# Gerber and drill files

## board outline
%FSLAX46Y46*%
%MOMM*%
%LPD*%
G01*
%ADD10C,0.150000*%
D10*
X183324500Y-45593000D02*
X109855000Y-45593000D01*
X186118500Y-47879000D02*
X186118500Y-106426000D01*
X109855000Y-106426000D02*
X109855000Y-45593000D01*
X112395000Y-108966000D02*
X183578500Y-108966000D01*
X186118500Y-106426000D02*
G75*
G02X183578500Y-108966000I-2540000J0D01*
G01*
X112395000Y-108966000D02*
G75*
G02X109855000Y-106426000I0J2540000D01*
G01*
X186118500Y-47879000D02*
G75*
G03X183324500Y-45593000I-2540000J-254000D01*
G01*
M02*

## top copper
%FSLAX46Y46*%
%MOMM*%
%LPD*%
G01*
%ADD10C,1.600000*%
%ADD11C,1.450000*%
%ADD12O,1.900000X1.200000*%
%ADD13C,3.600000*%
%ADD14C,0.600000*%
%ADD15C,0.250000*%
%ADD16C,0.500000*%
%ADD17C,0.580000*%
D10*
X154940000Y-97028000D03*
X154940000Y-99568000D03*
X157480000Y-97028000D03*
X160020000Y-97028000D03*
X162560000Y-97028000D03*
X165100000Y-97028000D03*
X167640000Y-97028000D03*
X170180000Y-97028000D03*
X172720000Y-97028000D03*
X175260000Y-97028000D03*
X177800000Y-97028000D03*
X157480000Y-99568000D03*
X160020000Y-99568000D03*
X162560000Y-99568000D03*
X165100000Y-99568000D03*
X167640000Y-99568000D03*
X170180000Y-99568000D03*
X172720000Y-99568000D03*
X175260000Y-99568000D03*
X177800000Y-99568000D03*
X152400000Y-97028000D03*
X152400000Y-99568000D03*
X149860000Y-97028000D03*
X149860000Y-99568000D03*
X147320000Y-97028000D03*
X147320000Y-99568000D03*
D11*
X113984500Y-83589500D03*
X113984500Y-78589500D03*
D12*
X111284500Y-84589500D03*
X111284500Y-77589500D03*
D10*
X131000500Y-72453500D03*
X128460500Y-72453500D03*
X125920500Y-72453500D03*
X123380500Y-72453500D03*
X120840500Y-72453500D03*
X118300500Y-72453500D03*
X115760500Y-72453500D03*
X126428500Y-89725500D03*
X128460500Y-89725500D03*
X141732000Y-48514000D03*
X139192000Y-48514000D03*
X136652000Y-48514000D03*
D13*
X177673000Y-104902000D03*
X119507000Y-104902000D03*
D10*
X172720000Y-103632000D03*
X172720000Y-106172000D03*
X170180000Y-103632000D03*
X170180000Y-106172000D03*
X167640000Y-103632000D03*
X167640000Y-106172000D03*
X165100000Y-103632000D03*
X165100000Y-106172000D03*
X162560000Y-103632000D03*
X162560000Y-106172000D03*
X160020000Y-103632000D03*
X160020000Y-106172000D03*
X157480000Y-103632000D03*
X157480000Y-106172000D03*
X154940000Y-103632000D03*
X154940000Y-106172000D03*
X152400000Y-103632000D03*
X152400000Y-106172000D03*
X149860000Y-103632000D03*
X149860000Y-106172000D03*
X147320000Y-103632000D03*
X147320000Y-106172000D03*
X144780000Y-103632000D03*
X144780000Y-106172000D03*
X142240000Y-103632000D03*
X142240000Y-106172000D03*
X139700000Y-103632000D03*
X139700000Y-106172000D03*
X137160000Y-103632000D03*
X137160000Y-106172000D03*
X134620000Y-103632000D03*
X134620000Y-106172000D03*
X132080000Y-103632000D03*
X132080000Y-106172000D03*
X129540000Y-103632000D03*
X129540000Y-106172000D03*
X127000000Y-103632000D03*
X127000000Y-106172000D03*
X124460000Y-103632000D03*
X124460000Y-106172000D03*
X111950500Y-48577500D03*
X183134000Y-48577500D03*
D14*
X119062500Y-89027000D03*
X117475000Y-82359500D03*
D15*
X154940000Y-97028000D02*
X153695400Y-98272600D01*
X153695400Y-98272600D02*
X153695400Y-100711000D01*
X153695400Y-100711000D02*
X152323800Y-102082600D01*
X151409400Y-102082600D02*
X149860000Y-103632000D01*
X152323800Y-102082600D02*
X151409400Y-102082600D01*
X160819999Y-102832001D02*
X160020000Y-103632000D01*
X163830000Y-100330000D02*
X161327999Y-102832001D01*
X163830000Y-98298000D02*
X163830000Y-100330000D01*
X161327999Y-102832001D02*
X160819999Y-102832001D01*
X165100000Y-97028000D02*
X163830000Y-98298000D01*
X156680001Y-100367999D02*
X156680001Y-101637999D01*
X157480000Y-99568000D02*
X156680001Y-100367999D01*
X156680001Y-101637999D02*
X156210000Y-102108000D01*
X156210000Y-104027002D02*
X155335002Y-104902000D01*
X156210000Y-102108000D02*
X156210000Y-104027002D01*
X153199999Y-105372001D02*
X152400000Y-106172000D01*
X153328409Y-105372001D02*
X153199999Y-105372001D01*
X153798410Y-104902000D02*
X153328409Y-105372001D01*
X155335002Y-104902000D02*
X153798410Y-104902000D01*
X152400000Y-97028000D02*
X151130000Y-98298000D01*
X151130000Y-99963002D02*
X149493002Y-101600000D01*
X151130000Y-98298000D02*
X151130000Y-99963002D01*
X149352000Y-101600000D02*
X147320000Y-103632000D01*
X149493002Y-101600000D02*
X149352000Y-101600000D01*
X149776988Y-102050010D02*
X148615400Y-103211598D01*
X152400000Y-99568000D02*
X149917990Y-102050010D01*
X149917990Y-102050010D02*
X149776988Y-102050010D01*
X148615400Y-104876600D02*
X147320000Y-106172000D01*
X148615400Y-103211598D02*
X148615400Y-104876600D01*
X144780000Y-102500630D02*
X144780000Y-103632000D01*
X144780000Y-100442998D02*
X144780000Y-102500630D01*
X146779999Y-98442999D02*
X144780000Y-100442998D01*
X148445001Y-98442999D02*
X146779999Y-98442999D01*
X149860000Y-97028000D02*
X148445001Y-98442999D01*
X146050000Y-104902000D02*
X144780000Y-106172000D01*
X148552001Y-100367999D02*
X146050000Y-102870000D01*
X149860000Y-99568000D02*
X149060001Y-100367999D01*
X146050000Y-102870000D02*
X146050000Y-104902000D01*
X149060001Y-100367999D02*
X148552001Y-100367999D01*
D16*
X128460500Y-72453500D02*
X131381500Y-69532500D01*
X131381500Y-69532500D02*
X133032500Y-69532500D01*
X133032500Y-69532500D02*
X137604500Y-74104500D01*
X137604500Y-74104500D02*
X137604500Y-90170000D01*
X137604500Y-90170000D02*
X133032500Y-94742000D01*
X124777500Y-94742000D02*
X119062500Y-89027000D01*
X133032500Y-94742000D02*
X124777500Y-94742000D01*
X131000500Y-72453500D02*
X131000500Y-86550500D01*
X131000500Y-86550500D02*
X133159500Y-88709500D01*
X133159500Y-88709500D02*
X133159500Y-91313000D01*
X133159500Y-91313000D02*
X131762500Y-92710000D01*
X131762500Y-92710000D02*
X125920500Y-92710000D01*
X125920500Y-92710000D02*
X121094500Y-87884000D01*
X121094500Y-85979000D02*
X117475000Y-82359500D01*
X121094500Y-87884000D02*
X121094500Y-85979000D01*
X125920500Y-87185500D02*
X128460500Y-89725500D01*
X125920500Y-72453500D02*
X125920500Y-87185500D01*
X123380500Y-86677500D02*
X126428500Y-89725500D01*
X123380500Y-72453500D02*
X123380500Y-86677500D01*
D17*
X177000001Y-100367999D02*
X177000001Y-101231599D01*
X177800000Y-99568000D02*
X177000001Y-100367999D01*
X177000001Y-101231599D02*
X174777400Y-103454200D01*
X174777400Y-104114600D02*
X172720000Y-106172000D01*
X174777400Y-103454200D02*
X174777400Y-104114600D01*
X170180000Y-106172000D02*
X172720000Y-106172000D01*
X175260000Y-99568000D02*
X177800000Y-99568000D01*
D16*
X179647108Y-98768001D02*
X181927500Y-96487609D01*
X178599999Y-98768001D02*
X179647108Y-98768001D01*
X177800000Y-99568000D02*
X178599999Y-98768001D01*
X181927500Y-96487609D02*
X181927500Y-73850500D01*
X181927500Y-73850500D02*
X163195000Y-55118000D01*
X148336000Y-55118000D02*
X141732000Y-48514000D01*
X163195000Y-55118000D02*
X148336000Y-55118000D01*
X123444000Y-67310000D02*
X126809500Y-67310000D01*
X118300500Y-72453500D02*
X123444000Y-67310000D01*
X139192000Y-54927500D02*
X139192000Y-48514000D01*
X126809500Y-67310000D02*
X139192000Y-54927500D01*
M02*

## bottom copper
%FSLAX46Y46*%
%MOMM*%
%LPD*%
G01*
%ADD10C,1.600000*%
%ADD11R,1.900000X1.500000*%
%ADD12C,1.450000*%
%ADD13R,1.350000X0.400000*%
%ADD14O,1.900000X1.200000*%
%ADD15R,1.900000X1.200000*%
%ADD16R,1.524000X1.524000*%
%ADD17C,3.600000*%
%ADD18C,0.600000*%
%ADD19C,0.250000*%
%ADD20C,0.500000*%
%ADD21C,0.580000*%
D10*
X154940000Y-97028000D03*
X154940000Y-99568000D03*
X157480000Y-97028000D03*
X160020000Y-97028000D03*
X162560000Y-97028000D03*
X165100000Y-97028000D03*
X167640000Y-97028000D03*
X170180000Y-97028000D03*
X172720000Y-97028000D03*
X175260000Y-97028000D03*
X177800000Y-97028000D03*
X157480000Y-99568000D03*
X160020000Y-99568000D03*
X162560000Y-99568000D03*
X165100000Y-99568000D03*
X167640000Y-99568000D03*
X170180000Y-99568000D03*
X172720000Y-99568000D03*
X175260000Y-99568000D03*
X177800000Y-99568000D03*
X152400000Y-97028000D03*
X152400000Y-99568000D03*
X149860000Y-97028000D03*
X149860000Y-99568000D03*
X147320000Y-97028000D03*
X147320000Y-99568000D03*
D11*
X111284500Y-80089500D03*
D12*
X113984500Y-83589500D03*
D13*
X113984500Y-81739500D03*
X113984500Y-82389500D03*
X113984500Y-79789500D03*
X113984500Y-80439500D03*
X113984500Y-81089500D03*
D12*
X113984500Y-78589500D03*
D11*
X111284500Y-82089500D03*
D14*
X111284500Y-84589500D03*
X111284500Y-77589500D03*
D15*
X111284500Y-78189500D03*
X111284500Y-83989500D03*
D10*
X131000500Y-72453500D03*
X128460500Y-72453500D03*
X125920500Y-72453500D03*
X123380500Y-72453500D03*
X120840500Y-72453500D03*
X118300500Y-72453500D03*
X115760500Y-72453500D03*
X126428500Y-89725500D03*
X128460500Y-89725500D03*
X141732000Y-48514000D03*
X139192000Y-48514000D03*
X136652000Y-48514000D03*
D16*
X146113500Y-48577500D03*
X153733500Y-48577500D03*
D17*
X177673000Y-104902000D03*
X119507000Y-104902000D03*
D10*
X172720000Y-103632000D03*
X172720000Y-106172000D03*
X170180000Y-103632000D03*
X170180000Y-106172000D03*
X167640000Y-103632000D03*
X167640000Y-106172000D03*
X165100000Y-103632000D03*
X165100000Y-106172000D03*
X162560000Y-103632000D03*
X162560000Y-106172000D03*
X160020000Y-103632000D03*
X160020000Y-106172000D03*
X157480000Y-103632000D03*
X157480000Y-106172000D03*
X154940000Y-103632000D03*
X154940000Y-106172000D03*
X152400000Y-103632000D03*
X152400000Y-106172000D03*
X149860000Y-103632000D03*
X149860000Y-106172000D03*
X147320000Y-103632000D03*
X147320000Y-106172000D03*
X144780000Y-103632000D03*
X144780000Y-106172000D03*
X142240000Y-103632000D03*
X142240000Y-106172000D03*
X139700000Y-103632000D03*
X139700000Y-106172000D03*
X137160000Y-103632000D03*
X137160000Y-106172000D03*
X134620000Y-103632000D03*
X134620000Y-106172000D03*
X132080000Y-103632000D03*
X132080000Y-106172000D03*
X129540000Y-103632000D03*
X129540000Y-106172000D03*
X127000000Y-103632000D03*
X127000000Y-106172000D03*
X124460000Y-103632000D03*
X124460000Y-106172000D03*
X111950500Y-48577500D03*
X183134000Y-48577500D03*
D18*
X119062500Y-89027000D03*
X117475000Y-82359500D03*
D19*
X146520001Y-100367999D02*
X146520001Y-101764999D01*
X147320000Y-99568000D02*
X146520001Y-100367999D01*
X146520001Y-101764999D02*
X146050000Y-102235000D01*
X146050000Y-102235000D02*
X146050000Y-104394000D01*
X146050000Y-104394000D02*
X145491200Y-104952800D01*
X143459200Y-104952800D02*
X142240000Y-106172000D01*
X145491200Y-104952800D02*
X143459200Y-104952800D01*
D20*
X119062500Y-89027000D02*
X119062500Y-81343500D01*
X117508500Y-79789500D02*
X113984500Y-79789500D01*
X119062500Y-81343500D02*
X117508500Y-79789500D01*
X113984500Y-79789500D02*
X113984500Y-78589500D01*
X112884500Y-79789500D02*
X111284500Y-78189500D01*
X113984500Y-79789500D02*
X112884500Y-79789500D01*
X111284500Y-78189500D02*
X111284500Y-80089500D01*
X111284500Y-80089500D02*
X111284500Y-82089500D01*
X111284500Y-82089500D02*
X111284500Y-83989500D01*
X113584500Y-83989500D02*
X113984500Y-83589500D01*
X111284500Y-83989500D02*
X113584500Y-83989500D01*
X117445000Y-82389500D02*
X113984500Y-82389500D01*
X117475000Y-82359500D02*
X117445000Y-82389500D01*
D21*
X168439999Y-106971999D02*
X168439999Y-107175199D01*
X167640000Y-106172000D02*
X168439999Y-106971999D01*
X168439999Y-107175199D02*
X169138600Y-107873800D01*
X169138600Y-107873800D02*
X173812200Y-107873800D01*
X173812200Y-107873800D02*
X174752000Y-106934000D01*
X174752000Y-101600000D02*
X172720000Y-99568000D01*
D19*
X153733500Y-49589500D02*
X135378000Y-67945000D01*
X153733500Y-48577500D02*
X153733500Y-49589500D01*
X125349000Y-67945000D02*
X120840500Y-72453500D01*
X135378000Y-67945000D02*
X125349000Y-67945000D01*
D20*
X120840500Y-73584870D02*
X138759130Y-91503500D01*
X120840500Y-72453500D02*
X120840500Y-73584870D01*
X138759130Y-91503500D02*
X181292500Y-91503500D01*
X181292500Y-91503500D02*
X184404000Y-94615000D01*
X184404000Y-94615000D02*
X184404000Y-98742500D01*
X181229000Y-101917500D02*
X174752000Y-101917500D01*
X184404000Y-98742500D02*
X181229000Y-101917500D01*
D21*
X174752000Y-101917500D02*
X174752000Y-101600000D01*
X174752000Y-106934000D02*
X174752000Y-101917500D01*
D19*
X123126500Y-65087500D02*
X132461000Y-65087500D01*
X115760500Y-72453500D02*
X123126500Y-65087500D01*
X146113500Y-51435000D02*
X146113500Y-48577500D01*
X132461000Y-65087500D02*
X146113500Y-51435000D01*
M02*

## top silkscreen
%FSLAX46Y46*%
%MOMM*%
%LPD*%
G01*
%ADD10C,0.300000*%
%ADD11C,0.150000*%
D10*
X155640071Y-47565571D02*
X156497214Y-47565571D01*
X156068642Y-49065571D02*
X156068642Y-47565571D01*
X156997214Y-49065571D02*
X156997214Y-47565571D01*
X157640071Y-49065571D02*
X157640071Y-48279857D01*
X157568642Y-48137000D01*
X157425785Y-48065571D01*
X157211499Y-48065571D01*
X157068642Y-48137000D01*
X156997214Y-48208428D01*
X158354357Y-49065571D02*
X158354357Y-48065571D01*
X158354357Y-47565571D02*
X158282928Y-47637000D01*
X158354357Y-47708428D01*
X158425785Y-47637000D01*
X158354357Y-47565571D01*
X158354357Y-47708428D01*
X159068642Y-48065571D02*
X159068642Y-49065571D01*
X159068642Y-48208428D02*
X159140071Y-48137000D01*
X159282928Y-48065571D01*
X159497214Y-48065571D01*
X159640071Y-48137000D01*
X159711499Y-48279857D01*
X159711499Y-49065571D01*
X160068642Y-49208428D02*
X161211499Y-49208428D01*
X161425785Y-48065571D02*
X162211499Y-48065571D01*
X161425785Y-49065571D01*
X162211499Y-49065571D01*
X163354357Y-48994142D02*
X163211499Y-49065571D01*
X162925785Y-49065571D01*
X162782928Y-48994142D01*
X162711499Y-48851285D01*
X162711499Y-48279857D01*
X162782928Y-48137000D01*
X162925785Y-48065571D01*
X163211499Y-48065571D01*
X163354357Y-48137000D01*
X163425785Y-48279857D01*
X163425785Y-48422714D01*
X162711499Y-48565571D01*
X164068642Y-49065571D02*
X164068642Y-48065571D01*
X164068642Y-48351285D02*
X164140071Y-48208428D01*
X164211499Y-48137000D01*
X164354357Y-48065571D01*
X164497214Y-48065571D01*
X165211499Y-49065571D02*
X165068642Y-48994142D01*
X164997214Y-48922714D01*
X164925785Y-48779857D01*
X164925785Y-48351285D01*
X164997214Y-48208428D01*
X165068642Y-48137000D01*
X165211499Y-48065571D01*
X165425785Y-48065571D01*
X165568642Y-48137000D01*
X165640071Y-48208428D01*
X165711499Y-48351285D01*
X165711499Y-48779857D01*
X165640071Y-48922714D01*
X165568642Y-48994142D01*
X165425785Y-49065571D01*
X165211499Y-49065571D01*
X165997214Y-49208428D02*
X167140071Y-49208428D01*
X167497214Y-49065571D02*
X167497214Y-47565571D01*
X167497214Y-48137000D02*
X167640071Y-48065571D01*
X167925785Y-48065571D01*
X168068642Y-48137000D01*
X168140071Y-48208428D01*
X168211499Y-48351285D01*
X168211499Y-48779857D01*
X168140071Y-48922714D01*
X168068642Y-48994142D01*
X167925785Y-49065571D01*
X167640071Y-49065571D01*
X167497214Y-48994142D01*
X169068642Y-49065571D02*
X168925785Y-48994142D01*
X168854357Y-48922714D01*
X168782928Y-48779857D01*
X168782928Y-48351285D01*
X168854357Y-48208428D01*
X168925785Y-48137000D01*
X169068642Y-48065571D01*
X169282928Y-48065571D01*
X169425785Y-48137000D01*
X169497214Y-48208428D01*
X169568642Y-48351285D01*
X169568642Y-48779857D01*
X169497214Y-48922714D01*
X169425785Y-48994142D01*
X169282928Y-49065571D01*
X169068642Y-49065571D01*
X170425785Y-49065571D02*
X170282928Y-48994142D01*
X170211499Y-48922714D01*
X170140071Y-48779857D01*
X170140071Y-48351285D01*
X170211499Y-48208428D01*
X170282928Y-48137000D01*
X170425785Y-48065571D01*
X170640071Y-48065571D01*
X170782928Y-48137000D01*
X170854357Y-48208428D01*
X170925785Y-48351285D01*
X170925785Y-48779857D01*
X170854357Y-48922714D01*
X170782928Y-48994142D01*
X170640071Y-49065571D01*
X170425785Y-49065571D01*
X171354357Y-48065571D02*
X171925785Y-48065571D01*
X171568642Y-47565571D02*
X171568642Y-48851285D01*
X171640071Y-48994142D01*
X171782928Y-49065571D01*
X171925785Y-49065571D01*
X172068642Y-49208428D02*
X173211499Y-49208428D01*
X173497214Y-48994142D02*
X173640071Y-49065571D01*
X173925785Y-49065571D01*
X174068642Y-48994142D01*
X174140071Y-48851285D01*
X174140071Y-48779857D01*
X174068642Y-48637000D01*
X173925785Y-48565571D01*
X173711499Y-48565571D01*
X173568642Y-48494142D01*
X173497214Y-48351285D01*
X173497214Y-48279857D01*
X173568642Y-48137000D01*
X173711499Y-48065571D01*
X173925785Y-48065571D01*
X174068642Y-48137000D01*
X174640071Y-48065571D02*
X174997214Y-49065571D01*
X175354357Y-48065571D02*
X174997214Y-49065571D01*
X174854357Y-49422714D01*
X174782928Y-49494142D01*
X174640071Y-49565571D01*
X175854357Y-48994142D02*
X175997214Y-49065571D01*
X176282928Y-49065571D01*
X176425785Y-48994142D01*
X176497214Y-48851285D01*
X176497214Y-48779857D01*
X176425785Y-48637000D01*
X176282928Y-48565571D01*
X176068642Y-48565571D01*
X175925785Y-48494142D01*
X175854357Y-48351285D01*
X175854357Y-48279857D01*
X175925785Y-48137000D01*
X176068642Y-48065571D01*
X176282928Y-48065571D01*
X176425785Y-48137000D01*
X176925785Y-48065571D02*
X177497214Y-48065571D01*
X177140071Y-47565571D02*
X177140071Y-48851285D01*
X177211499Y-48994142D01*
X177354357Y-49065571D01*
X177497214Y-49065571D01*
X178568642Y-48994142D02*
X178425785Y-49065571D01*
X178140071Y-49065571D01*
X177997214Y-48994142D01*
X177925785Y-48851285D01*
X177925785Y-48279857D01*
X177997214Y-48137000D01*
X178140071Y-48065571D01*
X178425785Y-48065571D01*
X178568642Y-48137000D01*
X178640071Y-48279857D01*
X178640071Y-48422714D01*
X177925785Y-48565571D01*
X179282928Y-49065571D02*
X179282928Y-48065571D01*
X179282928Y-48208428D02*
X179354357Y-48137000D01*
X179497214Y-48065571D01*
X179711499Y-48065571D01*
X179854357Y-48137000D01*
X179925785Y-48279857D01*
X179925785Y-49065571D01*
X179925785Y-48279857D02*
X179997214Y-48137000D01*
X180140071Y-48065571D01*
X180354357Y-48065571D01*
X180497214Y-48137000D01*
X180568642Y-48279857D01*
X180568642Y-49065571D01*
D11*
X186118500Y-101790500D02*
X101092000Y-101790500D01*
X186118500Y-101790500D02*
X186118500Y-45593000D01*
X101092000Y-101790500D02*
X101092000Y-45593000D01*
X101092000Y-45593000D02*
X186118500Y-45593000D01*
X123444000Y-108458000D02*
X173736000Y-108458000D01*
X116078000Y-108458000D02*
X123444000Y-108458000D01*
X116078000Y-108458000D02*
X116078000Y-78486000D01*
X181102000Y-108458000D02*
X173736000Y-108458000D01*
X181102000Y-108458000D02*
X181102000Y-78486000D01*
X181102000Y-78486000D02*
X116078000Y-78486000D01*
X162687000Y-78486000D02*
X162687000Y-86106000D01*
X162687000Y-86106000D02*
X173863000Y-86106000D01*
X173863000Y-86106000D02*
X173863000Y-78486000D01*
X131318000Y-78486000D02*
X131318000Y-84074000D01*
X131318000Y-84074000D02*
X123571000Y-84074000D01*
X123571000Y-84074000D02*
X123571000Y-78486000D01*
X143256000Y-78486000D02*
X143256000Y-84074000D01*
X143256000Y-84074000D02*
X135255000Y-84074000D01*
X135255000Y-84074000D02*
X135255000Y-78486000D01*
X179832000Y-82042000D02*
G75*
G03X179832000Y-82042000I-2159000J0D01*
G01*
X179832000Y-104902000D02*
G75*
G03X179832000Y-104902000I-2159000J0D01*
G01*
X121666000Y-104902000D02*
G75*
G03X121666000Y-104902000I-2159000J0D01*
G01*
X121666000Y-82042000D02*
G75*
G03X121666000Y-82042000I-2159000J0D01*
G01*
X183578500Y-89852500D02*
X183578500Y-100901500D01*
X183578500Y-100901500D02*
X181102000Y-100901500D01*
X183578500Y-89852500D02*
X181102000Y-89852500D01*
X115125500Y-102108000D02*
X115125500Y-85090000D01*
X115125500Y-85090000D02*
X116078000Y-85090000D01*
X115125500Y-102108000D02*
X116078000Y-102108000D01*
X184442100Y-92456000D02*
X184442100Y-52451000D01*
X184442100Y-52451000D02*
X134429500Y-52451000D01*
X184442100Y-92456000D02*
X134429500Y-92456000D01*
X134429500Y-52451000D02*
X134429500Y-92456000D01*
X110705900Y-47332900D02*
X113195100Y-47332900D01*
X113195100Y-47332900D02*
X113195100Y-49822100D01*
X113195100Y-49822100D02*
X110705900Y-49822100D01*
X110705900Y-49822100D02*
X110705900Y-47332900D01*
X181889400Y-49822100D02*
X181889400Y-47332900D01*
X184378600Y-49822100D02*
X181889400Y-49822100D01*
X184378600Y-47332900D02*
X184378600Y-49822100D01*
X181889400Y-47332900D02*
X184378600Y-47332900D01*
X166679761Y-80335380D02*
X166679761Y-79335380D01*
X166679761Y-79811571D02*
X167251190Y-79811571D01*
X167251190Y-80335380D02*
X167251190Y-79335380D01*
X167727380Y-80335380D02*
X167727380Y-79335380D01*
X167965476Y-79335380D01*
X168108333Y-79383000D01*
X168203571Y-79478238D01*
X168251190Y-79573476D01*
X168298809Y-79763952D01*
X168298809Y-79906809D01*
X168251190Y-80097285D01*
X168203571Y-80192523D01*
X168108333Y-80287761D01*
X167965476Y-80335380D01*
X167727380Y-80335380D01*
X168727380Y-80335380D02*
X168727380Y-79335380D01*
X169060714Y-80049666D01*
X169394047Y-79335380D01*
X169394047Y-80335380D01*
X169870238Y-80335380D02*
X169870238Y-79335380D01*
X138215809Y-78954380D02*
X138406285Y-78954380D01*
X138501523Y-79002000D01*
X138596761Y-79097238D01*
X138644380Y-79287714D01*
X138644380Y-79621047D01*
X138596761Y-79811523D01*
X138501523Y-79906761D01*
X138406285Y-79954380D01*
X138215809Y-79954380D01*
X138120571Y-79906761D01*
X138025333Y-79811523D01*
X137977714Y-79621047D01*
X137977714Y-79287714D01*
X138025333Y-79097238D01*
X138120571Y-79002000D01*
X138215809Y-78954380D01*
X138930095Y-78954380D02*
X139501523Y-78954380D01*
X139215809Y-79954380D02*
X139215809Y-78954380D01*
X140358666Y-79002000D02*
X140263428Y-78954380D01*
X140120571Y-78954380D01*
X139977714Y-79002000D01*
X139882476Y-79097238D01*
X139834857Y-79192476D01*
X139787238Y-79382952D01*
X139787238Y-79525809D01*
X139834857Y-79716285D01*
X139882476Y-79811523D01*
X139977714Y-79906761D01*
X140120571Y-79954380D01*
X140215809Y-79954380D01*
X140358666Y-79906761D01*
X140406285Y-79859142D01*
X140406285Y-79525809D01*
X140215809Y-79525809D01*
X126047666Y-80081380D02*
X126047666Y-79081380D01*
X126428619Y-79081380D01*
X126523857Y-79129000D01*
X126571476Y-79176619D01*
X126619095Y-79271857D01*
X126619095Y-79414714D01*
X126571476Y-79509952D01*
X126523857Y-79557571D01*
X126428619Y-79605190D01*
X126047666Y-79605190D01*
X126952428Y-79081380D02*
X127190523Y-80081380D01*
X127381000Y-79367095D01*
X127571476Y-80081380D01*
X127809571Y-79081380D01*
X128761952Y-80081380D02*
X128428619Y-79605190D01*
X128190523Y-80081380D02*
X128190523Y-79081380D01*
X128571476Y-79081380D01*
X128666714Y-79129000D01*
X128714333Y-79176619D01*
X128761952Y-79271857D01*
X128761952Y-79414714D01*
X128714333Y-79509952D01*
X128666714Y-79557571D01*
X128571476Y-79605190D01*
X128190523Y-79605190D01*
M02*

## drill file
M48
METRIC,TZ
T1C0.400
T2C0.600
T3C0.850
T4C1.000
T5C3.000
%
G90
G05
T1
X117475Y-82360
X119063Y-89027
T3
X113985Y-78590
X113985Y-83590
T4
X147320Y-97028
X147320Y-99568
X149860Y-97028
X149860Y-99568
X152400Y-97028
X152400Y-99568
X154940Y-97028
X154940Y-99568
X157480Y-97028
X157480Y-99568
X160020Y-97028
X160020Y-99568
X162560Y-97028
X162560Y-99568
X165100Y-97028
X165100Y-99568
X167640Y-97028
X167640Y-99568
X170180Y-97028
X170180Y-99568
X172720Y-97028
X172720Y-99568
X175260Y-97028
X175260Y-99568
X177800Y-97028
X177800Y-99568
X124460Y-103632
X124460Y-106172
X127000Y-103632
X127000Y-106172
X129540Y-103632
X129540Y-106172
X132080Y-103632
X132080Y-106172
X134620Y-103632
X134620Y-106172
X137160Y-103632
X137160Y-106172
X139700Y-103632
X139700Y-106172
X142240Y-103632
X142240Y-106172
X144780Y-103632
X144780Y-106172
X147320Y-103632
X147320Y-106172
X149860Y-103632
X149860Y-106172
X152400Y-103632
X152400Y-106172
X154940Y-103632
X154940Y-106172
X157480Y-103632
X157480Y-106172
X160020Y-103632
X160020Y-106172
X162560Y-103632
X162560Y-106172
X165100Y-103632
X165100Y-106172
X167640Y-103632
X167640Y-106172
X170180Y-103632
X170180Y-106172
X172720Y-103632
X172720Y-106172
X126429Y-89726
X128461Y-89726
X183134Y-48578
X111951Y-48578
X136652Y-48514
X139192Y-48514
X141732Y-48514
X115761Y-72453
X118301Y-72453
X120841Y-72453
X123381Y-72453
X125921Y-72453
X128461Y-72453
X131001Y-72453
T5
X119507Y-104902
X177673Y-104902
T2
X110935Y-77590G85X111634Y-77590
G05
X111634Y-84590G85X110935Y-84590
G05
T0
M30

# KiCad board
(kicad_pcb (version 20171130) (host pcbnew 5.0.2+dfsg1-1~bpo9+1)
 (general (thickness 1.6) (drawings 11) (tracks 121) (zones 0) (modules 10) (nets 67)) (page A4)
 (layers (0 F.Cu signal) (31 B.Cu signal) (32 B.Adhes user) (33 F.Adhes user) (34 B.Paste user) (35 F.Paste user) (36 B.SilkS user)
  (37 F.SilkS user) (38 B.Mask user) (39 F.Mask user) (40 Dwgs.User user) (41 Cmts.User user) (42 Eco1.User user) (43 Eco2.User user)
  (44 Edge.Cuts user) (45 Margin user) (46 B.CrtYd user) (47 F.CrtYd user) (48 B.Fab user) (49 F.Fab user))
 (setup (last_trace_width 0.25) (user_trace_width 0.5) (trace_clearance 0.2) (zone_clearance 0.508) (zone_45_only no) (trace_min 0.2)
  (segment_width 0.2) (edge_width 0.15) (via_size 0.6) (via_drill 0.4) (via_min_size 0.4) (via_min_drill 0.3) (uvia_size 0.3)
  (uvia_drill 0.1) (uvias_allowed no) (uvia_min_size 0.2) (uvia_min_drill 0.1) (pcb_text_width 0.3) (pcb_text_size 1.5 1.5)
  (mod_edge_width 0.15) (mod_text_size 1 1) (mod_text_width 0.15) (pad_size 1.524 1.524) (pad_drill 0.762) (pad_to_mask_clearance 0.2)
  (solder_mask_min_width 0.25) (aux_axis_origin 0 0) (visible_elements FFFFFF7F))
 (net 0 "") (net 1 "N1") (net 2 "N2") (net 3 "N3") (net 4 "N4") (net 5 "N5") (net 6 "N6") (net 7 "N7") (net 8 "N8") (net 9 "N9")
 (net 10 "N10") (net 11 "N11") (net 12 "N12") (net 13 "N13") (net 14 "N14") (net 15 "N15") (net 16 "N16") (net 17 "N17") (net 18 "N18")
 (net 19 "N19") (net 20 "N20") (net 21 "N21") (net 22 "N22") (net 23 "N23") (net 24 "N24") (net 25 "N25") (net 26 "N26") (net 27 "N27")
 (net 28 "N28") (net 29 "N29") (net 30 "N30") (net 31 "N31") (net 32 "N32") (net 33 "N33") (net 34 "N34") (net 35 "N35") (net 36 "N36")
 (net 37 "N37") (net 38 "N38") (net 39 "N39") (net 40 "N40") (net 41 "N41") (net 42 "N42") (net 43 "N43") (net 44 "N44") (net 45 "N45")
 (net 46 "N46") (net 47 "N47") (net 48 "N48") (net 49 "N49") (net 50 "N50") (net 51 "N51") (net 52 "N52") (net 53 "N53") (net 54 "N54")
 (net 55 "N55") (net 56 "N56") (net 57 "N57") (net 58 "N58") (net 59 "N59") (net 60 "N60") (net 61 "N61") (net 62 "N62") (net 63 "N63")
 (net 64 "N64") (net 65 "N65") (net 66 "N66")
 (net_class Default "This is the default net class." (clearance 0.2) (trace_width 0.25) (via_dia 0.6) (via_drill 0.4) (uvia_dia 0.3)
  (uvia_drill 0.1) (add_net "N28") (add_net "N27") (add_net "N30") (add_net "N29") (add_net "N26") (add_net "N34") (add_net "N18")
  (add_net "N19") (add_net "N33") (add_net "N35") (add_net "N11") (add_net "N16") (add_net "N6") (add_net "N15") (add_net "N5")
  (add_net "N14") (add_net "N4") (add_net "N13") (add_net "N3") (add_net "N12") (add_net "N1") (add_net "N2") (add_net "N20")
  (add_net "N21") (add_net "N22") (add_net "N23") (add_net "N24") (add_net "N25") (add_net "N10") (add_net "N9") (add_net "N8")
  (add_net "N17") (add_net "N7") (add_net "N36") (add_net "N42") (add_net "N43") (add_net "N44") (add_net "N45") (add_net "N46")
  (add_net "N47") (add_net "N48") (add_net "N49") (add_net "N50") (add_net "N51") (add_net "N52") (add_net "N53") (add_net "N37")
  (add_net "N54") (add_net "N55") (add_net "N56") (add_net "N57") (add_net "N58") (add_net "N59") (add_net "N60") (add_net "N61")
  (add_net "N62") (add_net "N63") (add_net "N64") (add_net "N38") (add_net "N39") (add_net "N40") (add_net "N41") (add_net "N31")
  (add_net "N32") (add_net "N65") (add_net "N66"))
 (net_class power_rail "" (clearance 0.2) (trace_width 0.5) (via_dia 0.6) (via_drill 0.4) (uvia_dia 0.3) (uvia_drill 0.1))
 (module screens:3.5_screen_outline (layer F.Cu) (at 162.56 98.298)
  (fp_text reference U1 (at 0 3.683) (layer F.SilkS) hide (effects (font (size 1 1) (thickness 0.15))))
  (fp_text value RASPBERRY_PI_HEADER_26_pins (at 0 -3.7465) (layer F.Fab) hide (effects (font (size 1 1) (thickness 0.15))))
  (fp_line (start 23.5585 3.4925) (end -61.468 3.4925) (layer F.SilkS) (width 0.15))
  (fp_line (start 23.5585 3.4925) (end 23.5585 -52.705) (layer F.SilkS) (width 0.15))
  (fp_line (start -61.468 3.4925) (end -61.468 -52.705) (layer F.SilkS) (width 0.15))
  (fp_line (start -61.468 -52.705) (end 23.5585 -52.705) (layer F.SilkS) (width 0.15))
  (pad 19 thru_hole circle (at -7.62 -1.27) (size 1.6 1.6) (drill 1) (layers *.Cu *.Mask) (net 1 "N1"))
  (pad 20 thru_hole circle (at -7.62 1.27) (size 1.6 1.6) (drill 1) (layers *.Cu *.Mask) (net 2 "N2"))
  (pad 17 thru_hole circle (at -5.08 -1.27) (size 1.6 1.6) (drill 1) (layers *.Cu *.Mask) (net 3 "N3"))
  (pad 15 thru_hole circle (at -2.54 -1.27) (size 1.6 1.6) (drill 1) (layers *.Cu *.Mask) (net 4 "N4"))
  (pad 13 thru_hole circle (at 0 -1.27) (size 1.6 1.6) (drill 1) (layers *.Cu *.Mask) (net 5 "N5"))
  (pad 11 thru_hole circle (at 2.54 -1.27) (size 1.6 1.6) (drill 1) (layers *.Cu *.Mask) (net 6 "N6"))
  (pad 9 thru_hole circle (at 5.08 -1.27) (size 1.6 1.6) (drill 1) (layers *.Cu *.Mask) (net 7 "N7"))
  (pad 7 thru_hole circle (at 7.62 -1.27) (size 1.6 1.6) (drill 1) (layers *.Cu *.Mask) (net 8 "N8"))
  (pad 5 thru_hole circle (at 10.16 -1.27) (size 1.6 1.6) (drill 1) (layers *.Cu *.Mask) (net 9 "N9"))
  (pad 3 thru_hole circle (at 12.7 -1.27) (size 1.6 1.6) (drill 1) (layers *.Cu *.Mask) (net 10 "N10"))
  (pad 1 thru_hole circle (at 15.24 -1.27) (size 1.6 1.6) (drill 1) (layers *.Cu *.Mask) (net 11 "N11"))
  (pad 18 thru_hole circle (at -5.08 1.27) (size 1.6 1.6) (drill 1) (layers *.Cu *.Mask) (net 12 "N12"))
  (pad 16 thru_hole circle (at -2.54 1.27) (size 1.6 1.6) (drill 1) (layers *.Cu *.Mask) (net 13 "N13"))
  (pad 14 thru_hole circle (at 0 1.27) (size 1.6 1.6) (drill 1) (layers *.Cu *.Mask) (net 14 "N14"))
  (pad 12 thru_hole circle (at 2.54 1.27) (size 1.6 1.6) (drill 1) (layers *.Cu *.Mask) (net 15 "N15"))
  (pad 10 thru_hole circle (at 5.08 1.27) (size 1.6 1.6) (drill 1) (layers *.Cu *.Mask) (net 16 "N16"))
  (pad 8 thru_hole circle (at 7.62 1.27) (size 1.6 1.6) (drill 1) (layers *.Cu *.Mask) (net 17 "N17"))
  (pad 6 thru_hole circle (at 10.16 1.27) (size 1.6 1.6) (drill 1) (layers *.Cu *.Mask) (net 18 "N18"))
  (pad 4 thru_hole circle (at 12.7 1.27) (size 1.6 1.6) (drill 1) (layers *.Cu *.Mask) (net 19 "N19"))
  (pad 2 thru_hole circle (at 15.24 1.27) (size 1.6 1.6) (drill 1) (layers *.Cu *.Mask) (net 19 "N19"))
  (pad 21 thru_hole circle (at -10.16 -1.27) (size 1.6 1.6) (drill 1) (layers *.Cu *.Mask) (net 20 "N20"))
  (pad 22 thru_hole circle (at -10.16 1.27) (size 1.6 1.6) (drill 1) (layers *.Cu *.Mask) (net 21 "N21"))
  (pad 23 thru_hole circle (at -12.7 -1.27) (size 1.6 1.6) (drill 1) (layers *.Cu *.Mask) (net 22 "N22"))
  (pad 24 thru_hole circle (at -12.7 1.27) (size 1.6 1.6) (drill 1) (layers *.Cu *.Mask) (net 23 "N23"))
  (pad 25 thru_hole circle (at -15.24 -1.27) (size 1.6 1.6) (drill 1) (layers *.Cu *.Mask) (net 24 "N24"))
  (pad 26 thru_hole circle (at -15.24 1.27) (size 1.6 1.6) (drill 1) (layers *.Cu *.Mask) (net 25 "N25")))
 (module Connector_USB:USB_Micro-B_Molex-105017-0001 (layer B.Cu) (at 112.522 81.0895 90)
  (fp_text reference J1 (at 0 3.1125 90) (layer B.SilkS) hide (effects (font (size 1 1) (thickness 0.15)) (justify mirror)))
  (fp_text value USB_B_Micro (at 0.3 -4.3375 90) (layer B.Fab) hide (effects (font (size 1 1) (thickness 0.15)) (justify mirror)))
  (pad 6 smd rect (at 1 -1.2375 90) (size 1.5 1.9) (layers B.Cu B.Paste B.Mask) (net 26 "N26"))
  (pad 6 thru_hole circle (at -2.5 1.4625 90) (size 1.45 1.45) (drill 0.85) (layers *.Cu *.Mask) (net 26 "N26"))
  (pad 2 smd rect (at -0.65 1.4625 90) (size 0.4 1.35) (layers B.Cu B.Paste B.Mask) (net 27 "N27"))
  (pad 1 smd rect (at -1.3 1.4625 90) (size 0.4 1.35) (layers B.Cu B.Paste B.Mask) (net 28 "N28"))
  (pad 5 smd rect (at 1.3 1.4625 90) (size 0.4 1.35) (layers B.Cu B.Paste B.Mask) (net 26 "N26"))
  (pad 4 smd rect (at 0.65 1.4625 90) (size 0.4 1.35) (layers B.Cu B.Paste B.Mask) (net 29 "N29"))
  (pad 3 smd rect (at 0 1.4625 90) (size 0.4 1.35) (layers B.Cu B.Paste B.Mask) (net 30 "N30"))
  (pad 6 thru_hole circle (at 2.5 1.4625 90) (size 1.45 1.45) (drill 0.85) (layers *.Cu *.Mask) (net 26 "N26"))
  (pad 6 smd rect (at -1 -1.2375 90) (size 1.5 1.9) (layers B.Cu B.Paste B.Mask) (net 26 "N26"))
  (pad 6 thru_hole oval (at -3.5 -1.2375 270) (size 1.2 1.9) (drill oval 0.6 1.3) (layers *.Cu *.Mask) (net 26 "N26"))
  (pad 6 thru_hole oval (at 3.5 -1.2375 90) (size 1.2 1.9) (drill oval 0.6 1.3) (layers *.Cu *.Mask) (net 26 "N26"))
  (pad 6 smd rect (at 2.9 -1.2375 90) (size 1.2 1.9) (layers B.Cu B.Mask) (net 26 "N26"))
  (pad 6 smd rect (at -2.9 -1.2375 90) (size 1.2 1.9) (layers B.Cu B.Mask) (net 26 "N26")))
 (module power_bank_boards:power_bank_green (layer B.Cu) (at 123.3805 72.4535 180)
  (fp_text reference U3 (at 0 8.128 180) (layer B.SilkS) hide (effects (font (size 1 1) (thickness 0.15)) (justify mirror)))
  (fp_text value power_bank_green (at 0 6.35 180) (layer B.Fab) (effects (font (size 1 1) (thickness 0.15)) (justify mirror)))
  (pad 1 thru_hole circle (at -7.62 0 180) (size 1.6 1.6) (drill 1) (layers *.Cu *.Mask) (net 28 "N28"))
  (pad 2 thru_hole circle (at -5.08 0 180) (size 1.6 1.6) (drill 1) (layers *.Cu *.Mask) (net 26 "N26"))
  (pad 3 thru_hole circle (at -2.54 0 180) (size 1.6 1.6) (drill 1) (layers *.Cu *.Mask) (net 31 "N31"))
  (pad 4 thru_hole circle (at 0 0 180) (size 1.6 1.6) (drill 1) (layers *.Cu *.Mask) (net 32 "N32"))
  (pad 5 thru_hole circle (at 2.54 0 180) (size 1.6 1.6) (drill 1) (layers *.Cu *.Mask) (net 18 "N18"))
  (pad 6 thru_hole circle (at 5.08 0 180) (size 1.6 1.6) (drill 1) (layers *.Cu *.Mask) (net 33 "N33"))
  (pad 7 thru_hole circle (at 7.62 0 180) (size 1.6 1.6) (drill 1) (layers *.Cu *.Mask) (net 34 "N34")))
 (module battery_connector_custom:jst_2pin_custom (layer B.Cu) (at 127.4445 89.7255)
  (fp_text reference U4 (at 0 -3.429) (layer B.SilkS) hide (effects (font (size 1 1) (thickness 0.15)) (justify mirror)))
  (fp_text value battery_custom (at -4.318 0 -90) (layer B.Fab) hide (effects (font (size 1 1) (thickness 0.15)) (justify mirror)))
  (pad 1 thru_hole circle (at -1.016 0) (size 1.6 1.6) (drill 1) (layers *.Cu *.Mask) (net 32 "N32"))
  (pad 2 thru_hole circle (at 1.016 0) (size 1.6 1.6) (drill 1) (layers *.Cu *.Mask) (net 31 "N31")))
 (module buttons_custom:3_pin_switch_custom (layer B.Cu) (at 139.192 48.514 180)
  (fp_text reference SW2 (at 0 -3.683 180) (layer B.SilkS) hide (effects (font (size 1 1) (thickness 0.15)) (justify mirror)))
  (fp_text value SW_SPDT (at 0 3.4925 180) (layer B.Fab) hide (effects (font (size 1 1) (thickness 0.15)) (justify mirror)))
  (pad 1 thru_hole circle (at -2.54 0 180) (size 1.6 1.6) (drill 1) (layers *.Cu *.Mask) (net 19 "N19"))
  (pad 2 thru_hole circle (at 0 0 180) (size 1.6 1.6) (drill 1) (layers *.Cu *.Mask) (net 33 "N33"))
  (pad 3 thru_hole circle (at 2.54 0 180) (size 1.6 1.6) (drill 1) (layers *.Cu *.Mask) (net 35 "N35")))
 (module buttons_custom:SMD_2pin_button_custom (layer B.Cu) (at 149.9235 48.5775 180)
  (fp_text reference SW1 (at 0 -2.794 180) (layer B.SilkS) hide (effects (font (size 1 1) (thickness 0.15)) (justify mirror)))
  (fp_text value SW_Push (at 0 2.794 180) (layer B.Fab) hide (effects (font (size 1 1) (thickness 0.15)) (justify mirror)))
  (pad 1 smd rect (at 3.81 0 180) (size 1.524 1.524) (layers B.Cu B.Paste B.Mask) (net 34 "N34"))
  (pad 2 smd rect (at -3.81 0 180) (size 1.524 1.524) (layers B.Cu B.Paste B.Mask) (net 18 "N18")))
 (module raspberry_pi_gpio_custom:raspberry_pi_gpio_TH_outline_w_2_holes (layer F.Cu) (at 148.59 104.902)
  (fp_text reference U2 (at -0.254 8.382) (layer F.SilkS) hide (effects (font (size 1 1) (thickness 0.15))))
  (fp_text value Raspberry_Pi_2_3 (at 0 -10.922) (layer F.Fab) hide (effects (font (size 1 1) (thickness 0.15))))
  (fp_line (start -25.146 3.556) (end 25.146 3.556) (layer F.SilkS) (width 0.15))
  (fp_line (start -32.512 3.556) (end -25.146 3.556) (layer F.SilkS) (width 0.15))
  (fp_line (start -32.512 3.556) (end -32.512 -26.416) (layer F.SilkS) (width 0.15))
  (fp_line (start 32.512 3.556) (end 25.146 3.556) (layer F.SilkS) (width 0.15))
  (fp_line (start 32.512 3.556) (end 32.512 -26.416) (layer F.SilkS) (width 0.15))
  (fp_line (start 32.512 -26.416) (end -32.512 -26.416) (layer F.SilkS) (width 0.15))
  (fp_line (start 14.097 -26.416) (end 14.097 -18.796) (layer F.SilkS) (width 0.15))
  (fp_line (start 14.097 -18.796) (end 25.273 -18.796) (layer F.SilkS) (width 0.15))
  (fp_line (start 25.273 -18.796) (end 25.273 -26.416) (layer F.SilkS) (width 0.15))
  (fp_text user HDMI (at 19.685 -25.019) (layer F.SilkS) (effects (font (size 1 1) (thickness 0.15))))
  (fp_line (start -17.272 -26.416) (end -17.272 -20.828) (layer F.SilkS) (width 0.15))
  (fp_line (start -17.272 -20.828) (end -25.019 -20.828) (layer F.SilkS) (width 0.15))
  (fp_line (start -25.019 -20.828) (end -25.019 -26.416) (layer F.SilkS) (width 0.15))
  (fp_line (start -5.334 -26.416) (end -5.334 -20.828) (layer F.SilkS) (width 0.15))
  (fp_line (start -5.334 -20.828) (end -13.335 -20.828) (layer F.SilkS) (width 0.15))
  (fp_line (start -13.335 -20.828) (end -13.335 -26.416) (layer F.SilkS) (width 0.15))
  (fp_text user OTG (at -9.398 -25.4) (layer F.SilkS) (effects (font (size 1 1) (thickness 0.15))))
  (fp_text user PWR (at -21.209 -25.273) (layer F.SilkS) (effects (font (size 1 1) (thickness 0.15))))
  (fp_circle (center 29.083 -22.86) (end 31.242 -22.86) (layer F.SilkS) (width 0.15))
  (fp_circle (center 29.083 0) (end 31.242 0) (layer F.SilkS) (width 0.15))
  (fp_circle (center -29.083 0) (end -26.924 0) (layer F.SilkS) (width 0.15))
  (fp_circle (center -29.083 -22.86) (end -26.924 -22.86) (layer F.SilkS) (width 0.15))
  (fp_line (start 34.9885 -15.0495) (end 34.9885 -4.0005) (layer F.SilkS) (width 0.15))
  (fp_line (start 34.9885 -4.0005) (end 32.512 -4.0005) (layer F.SilkS) (width 0.15))
  (fp_line (start 34.9885 -15.0495) (end 32.512 -15.0495) (layer F.SilkS) (width 0.15))
  (fp_line (start -33.4645 -2.794) (end -33.4645 -19.812) (layer F.SilkS) (width 0.15))
  (fp_line (start -33.4645 -19.812) (end -32.512 -19.812) (layer F.SilkS) (width 0.15))
  (fp_line (start -33.4645 -2.794) (end -32.512 -2.794) (layer F.SilkS) (width 0.15))
  (pad 0 thru_hole circle (at 29.083 0) (size 3.6 3.6) (drill 3) (layers *.Cu *.Mask))
  (pad 0 thru_hole circle (at -29.083 0) (size 3.6 3.6) (drill 3) (layers *.Cu *.Mask))
  (pad 1 thru_hole circle (at 24.13 -1.27 180) (size 1.6 1.6) (drill 1) (layers *.Cu *.Mask) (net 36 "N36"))
  (pad 2 thru_hole circle (at 24.13 1.27 180) (size 1.6 1.6) (drill 1) (layers *.Cu *.Mask) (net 19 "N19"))
  (pad 3 thru_hole circle (at 21.59 -1.27 180) (size 1.6 1.6) (drill 1) (layers *.Cu *.Mask) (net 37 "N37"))
  (pad 4 thru_hole circle (at 21.59 1.27 180) (size 1.6 1.6) (drill 1) (layers *.Cu *.Mask) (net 19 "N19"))
  (pad 5 thru_hole circle (at 19.05 -1.27 180) (size 1.6 1.6) (drill 1) (layers *.Cu *.Mask) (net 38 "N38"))
  (pad 6 thru_hole circle (at 19.05 1.27 180) (size 1.6 1.6) (drill 1) (layers *.Cu *.Mask) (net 18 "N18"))
  (pad 7 thru_hole circle (at 16.51 -1.27 180) (size 1.6 1.6) (drill 1) (layers *.Cu *.Mask) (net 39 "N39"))
  (pad 8 thru_hole circle (at 16.51 1.27 180) (size 1.6 1.6) (drill 1) (layers *.Cu *.Mask) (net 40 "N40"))
  (pad 9 thru_hole circle (at 13.97 -1.27 180) (size 1.6 1.6) (drill 1) (layers *.Cu *.Mask) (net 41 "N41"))
  (pad 10 thru_hole circle (at 13.97 1.27 180) (size 1.6 1.6) (drill 1) (layers *.Cu *.Mask) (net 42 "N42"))
  (pad 11 thru_hole circle (at 11.43 -1.27 180) (size 1.6 1.6) (drill 1) (layers *.Cu *.Mask) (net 6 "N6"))
  (pad 12 thru_hole circle (at 11.43 1.27 180) (size 1.6 1.6) (drill 1) (layers *.Cu *.Mask) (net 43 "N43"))
  (pad 13 thru_hole circle (at 8.89 -1.27 180) (size 1.6 1.6) (drill 1) (layers *.Cu *.Mask) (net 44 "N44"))
  (pad 14 thru_hole circle (at 8.89 1.27 180) (size 1.6 1.6) (drill 1) (layers *.Cu *.Mask) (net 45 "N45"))
  (pad 15 thru_hole circle (at 6.35 -1.27 180) (size 1.6 1.6) (drill 1) (layers *.Cu *.Mask) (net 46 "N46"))
  (pad 16 thru_hole circle (at 6.35 1.27 180) (size 1.6 1.6) (drill 1) (layers *.Cu *.Mask) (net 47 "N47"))
  (pad 17 thru_hole circle (at 3.81 -1.27 180) (size 1.6 1.6) (drill 1) (layers *.Cu *.Mask) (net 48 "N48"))
  (pad 18 thru_hole circle (at 3.81 1.27 180) (size 1.6 1.6) (drill 1) (layers *.Cu *.Mask) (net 12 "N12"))
  (pad 19 thru_hole circle (at 1.27 -1.27 180) (size 1.6 1.6) (drill 1) (layers *.Cu *.Mask) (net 1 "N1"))
  (pad 20 thru_hole circle (at 1.27 1.27 180) (size 1.6 1.6) (drill 1) (layers *.Cu *.Mask) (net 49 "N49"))
  (pad 21 thru_hole circle (at -1.27 -1.27 180) (size 1.6 1.6) (drill 1) (layers *.Cu *.Mask) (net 20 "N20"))
  (pad 22 thru_hole circle (at -1.27 1.27 180) (size 1.6 1.6) (drill 1) (layers *.Cu *.Mask) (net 21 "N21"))
  (pad 23 thru_hole circle (at -3.81 -1.27 180) (size 1.6 1.6) (drill 1) (layers *.Cu *.Mask) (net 22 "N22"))
  (pad 24 thru_hole circle (at -3.81 1.27 180) (size 1.6 1.6) (drill 1) (layers *.Cu *.Mask) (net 23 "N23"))
  (pad 25 thru_hole circle (at -6.35 -1.27 180) (size 1.6 1.6) (drill 1) (layers *.Cu *.Mask) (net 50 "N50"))
  (pad 26 thru_hole circle (at -6.35 1.27 180) (size 1.6 1.6) (drill 1) (layers *.Cu *.Mask) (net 25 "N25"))
  (pad 27 thru_hole circle (at -8.89 -1.27 180) (size 1.6 1.6) (drill 1) (layers *.Cu *.Mask) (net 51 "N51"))
  (pad 28 thru_hole circle (at -8.89 1.27 180) (size 1.6 1.6) (drill 1) (layers *.Cu *.Mask) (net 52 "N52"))
  (pad 29 thru_hole circle (at -11.43 -1.27 180) (size 1.6 1.6) (drill 1) (layers *.Cu *.Mask) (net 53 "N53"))
  (pad 30 thru_hole circle (at -11.43 1.27 180) (size 1.6 1.6) (drill 1) (layers *.Cu *.Mask) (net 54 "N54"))
  (pad 31 thru_hole circle (at -13.97 -1.27 180) (size 1.6 1.6) (drill 1) (layers *.Cu *.Mask) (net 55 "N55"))
  (pad 32 thru_hole circle (at -13.97 1.27 180) (size 1.6 1.6) (drill 1) (layers *.Cu *.Mask) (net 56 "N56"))
  (pad 33 thru_hole circle (at -16.51 -1.27 180) (size 1.6 1.6) (drill 1) (layers *.Cu *.Mask) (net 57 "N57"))
  (pad 34 thru_hole circle (at -16.51 1.27 180) (size 1.6 1.6) (drill 1) (layers *.Cu *.Mask) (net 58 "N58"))
  (pad 35 thru_hole circle (at -19.05 -1.27 180) (size 1.6 1.6) (drill 1) (layers *.Cu *.Mask) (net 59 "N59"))
  (pad 36 thru_hole circle (at -19.05 1.27 180) (size 1.6 1.6) (drill 1) (layers *.Cu *.Mask) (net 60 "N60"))
  (pad 37 thru_hole circle (at -21.59 -1.27 180) (size 1.6 1.6) (drill 1) (layers *.Cu *.Mask) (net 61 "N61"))
  (pad 38 thru_hole circle (at -21.59 1.27 180) (size 1.6 1.6) (drill 1) (layers *.Cu *.Mask) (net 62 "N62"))
  (pad 39 thru_hole circle (at -24.13 -1.27 180) (size 1.6 1.6) (drill 1) (layers *.Cu *.Mask) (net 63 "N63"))
  (pad 40 thru_hole circle (at -24.13 1.27 180) (size 1.6 1.6) (drill 1) (layers *.Cu *.Mask) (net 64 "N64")))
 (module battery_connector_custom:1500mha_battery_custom (layer F.Cu) (at 134.4295 92.456)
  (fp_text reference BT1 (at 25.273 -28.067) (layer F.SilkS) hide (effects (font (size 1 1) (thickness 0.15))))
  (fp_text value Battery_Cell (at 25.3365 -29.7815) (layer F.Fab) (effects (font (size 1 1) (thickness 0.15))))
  (fp_line (start 50.0126 0) (end 50.0126 -40.005) (layer F.SilkS) (width 0.15))
  (fp_line (start 50.0126 -40.005) (end 0 -40.005) (layer F.SilkS) (width 0.15))
  (fp_line (start 50.0126 0) (end 0 0) (layer F.SilkS) (width 0.15))
  (fp_line (start 0 -40.005) (end 0 0) (layer F.SilkS) (width 0.15)))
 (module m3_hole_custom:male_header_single (layer F.Cu) (at 111.9505 48.5775)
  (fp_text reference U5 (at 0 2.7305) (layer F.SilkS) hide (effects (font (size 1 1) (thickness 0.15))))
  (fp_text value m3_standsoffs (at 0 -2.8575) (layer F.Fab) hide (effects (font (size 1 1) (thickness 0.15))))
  (fp_line (start -1.2446 -1.2446) (end 1.2446 -1.2446) (layer F.SilkS) (width 0.15))
  (fp_line (start 1.2446 -1.2446) (end 1.2446 1.2446) (layer F.SilkS) (width 0.15))
  (fp_line (start 1.2446 1.2446) (end -1.2446 1.2446) (layer F.SilkS) (width 0.15))
  (fp_line (start -1.2446 1.2446) (end -1.2446 -1.2446) (layer F.SilkS) (width 0.15))
  (pad 1 thru_hole circle (at 0 0) (size 1.6 1.6) (drill 1) (layers *.Cu *.Mask) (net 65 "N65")))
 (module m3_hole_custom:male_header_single (layer F.Cu) (at 183.134 48.5775)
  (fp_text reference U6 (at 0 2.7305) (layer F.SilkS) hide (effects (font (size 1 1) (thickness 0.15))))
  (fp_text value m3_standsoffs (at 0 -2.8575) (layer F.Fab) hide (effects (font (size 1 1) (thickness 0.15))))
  (fp_line (start -1.2446 1.2446) (end -1.2446 -1.2446) (layer F.SilkS) (width 0.15))
  (fp_line (start 1.2446 1.2446) (end -1.2446 1.2446) (layer F.SilkS) (width 0.15))
  (fp_line (start 1.2446 -1.2446) (end 1.2446 1.2446) (layer F.SilkS) (width 0.15))
  (fp_line (start -1.2446 -1.2446) (end 1.2446 -1.2446) (layer F.SilkS) (width 0.15))
  (pad 1 thru_hole circle (at 0 0) (size 1.6 1.6) (drill 1) (layers *.Cu *.Mask) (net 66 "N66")))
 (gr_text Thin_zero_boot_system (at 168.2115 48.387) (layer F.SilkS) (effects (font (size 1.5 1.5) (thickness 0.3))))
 (gr_line (start 183.3245 45.593) (end 109.855 45.593) (layer Edge.Cuts) (width 0.15))
 (gr_line (start 186.1185 47.879) (end 186.1185 106.426) (layer Edge.Cuts) (width 0.15))
 (gr_line (start 109.855 106.426) (end 109.855 45.593) (layer Edge.Cuts) (width 0.15))
 (gr_line (start 112.395 108.966) (end 183.5785 108.966) (layer Edge.Cuts) (width 0.15))
 (gr_arc (start 183.5785 106.426) (end 183.5785 108.966) (angle -90) (layer Edge.Cuts) (width 0.15))
 (gr_arc (start 112.395 106.426) (end 109.855 106.426) (angle -90) (layer Edge.Cuts) (width 0.15))
 (gr_arc (start 183.5785 48.133) (end 183.3245 45.593) (angle 90) (layer Edge.Cuts) (width 0.15))
 (segment (start 154.94 97.028) (end 153.6954 98.2726) (width 0.25) (layer F.Cu) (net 1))
 (segment (start 153.6954 98.2726) (end 153.6954 100.711) (width 0.25) (layer F.Cu) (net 1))
 (segment (start 153.6954 100.711) (end 152.3238 102.0826) (width 0.25) (layer F.Cu) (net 1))
 (segment (start 151.4094 102.0826) (end 149.86 103.632) (width 0.25) (layer F.Cu) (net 1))
 (segment (start 152.3238 102.0826) (end 151.4094 102.0826) (width 0.25) (layer F.Cu) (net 1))
 (segment (start 160.819999 102.832001) (end 160.02 103.632) (width 0.25) (layer F.Cu) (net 6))
 (segment (start 163.83 100.33) (end 161.327999 102.832001) (width 0.25) (layer F.Cu) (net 6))
 (segment (start 163.83 98.298) (end 163.83 100.33) (width 0.25) (layer F.Cu) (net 6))
 (segment (start 161.327999 102.832001) (end 160.819999 102.832001) (width 0.25) (layer F.Cu) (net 6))
 (segment (start 165.1 97.028) (end 163.83 98.298) (width 0.25) (layer F.Cu) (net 6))
 (segment (start 156.680001 100.367999) (end 156.680001 101.637999) (width 0.25) (layer F.Cu) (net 12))
 (segment (start 157.48 99.568) (end 156.680001 100.367999) (width 0.25) (layer F.Cu) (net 12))
 (segment (start 156.680001 101.637999) (end 156.21 102.108) (width 0.25) (layer F.Cu) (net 12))
 (segment (start 156.21 104.027002) (end 155.335002 104.902) (width 0.25) (layer F.Cu) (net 12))
 (segment (start 156.21 102.108) (end 156.21 104.027002) (width 0.25) (layer F.Cu) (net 12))
 (segment (start 153.199999 105.372001) (end 152.4 106.172) (width 0.25) (layer F.Cu) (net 12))
 (segment (start 153.328409 105.372001) (end 153.199999 105.372001) (width 0.25) (layer F.Cu) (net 12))
 (segment (start 153.79841 104.902) (end 153.328409 105.372001) (width 0.25) (layer F.Cu) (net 12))
 (segment (start 155.335002 104.902) (end 153.79841 104.902) (width 0.25) (layer F.Cu) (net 12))
 (segment (start 152.4 97.028) (end 151.13 98.298) (width 0.25) (layer F.Cu) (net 20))
 (segment (start 151.13 99.963002) (end 149.493002 101.6) (width 0.25) (layer F.Cu) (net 20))
 (segment (start 151.13 98.298) (end 151.13 99.963002) (width 0.25) (layer F.Cu) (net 20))
 (segment (start 149.352 101.6) (end 147.32 103.632) (width 0.25) (layer F.Cu) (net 20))
 (segment (start 149.493002 101.6) (end 149.352 101.6) (width 0.25) (layer F.Cu) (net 20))
 (segment (start 149.776988 102.05001) (end 148.6154 103.211598) (width 0.25) (layer F.Cu) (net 21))
 (segment (start 152.4 99.568) (end 149.91799 102.05001) (width 0.25) (layer F.Cu) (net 21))
 (segment (start 149.91799 102.05001) (end 149.776988 102.05001) (width 0.25) (layer F.Cu) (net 21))
 (segment (start 148.6154 104.8766) (end 147.32 106.172) (width 0.25) (layer F.Cu) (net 21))
 (segment (start 148.6154 103.211598) (end 148.6154 104.8766) (width 0.25) (layer F.Cu) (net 21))
 (segment (start 144.78 102.50063) (end 144.78 103.632) (width 0.25) (layer F.Cu) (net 22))
 (segment (start 144.78 100.442998) (end 144.78 102.50063) (width 0.25) (layer F.Cu) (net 22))
 (segment (start 146.779999 98.442999) (end 144.78 100.442998) (width 0.25) (layer F.Cu) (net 22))
 (segment (start 148.445001 98.442999) (end 146.779999 98.442999) (width 0.25) (layer F.Cu) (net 22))
 (segment (start 149.86 97.028) (end 148.445001 98.442999) (width 0.25) (layer F.Cu) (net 22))
 (segment (start 146.05 104.902) (end 144.78 106.172) (width 0.25) (layer F.Cu) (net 23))
 (segment (start 148.552001 100.367999) (end 146.05 102.87) (width 0.25) (layer F.Cu) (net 23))
 (segment (start 149.86 99.568) (end 149.060001 100.367999) (width 0.25) (layer F.Cu) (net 23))
 (segment (start 146.05 102.87) (end 146.05 104.902) (width 0.25) (layer F.Cu) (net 23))
 (segment (start 149.060001 100.367999) (end 148.552001 100.367999) (width 0.25) (layer F.Cu) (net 23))
 (segment (start 146.520001 100.367999) (end 146.520001 101.764999) (width 0.25) (layer B.Cu) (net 25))
 (segment (start 147.32 99.568) (end 146.520001 100.367999) (width 0.25) (layer B.Cu) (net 25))
 (segment (start 146.520001 101.764999) (end 146.05 102.235) (width 0.25) (layer B.Cu) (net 25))
 (segment (start 146.05 102.235) (end 146.05 104.394) (width 0.25) (layer B.Cu) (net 25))
 (segment (start 146.05 104.394) (end 145.4912 104.9528) (width 0.25) (layer B.Cu) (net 25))
 (segment (start 143.4592 104.9528) (end 142.24 106.172) (width 0.25) (layer B.Cu) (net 25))
 (segment (start 145.4912 104.9528) (end 143.4592 104.9528) (width 0.25) (layer B.Cu) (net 25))
 (segment (start 128.4605 72.4535) (end 131.3815 69.5325) (width 0.5) (layer F.Cu) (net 26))
 (segment (start 131.3815 69.5325) (end 133.0325 69.5325) (width 0.5) (layer F.Cu) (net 26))
 (segment (start 133.0325 69.5325) (end 137.6045 74.1045) (width 0.5) (layer F.Cu) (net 26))
 (segment (start 137.6045 74.1045) (end 137.6045 90.17) (width 0.5) (layer F.Cu) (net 26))
 (segment (start 137.6045 90.17) (end 133.0325 94.742) (width 0.5) (layer F.Cu) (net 26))
 (via (at 119.0625 89.027) (size 0.6) (drill 0.4) (layers F.Cu B.Cu) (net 26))
 (segment (start 124.7775 94.742) (end 119.0625 89.027) (width 0.5) (layer F.Cu) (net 26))
 (segment (start 133.0325 94.742) (end 124.7775 94.742) (width 0.5) (layer F.Cu) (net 26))
 (segment (start 119.0625 89.027) (end 119.0625 81.3435) (width 0.5) (layer B.Cu) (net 26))
 (segment (start 117.5085 79.7895) (end 113.9845 79.7895) (width 0.5) (layer B.Cu) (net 26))
 (segment (start 119.0625 81.3435) (end 117.5085 79.7895) (width 0.5) (layer B.Cu) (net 26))
 (segment (start 113.9845 79.7895) (end 113.9845 78.5895) (width 0.5) (layer B.Cu) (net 26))
 (segment (start 112.8845 79.7895) (end 111.2845 78.1895) (width 0.5) (layer B.Cu) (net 26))
 (segment (start 113.9845 79.7895) (end 112.8845 79.7895) (width 0.5) (layer B.Cu) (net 26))
 (segment (start 111.2845 78.1895) (end 111.2845 80.0895) (width 0.5) (layer B.Cu) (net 26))
 (segment (start 111.2845 80.0895) (end 111.2845 82.0895) (width 0.5) (layer B.Cu) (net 26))
 (segment (start 111.2845 82.0895) (end 111.2845 83.9895) (width 0.5) (layer B.Cu) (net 26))
 (segment (start 113.5845 83.9895) (end 113.9845 83.5895) (width 0.5) (layer B.Cu) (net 26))
 (segment (start 111.2845 83.9895) (end 113.5845 83.9895) (width 0.5) (layer B.Cu) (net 26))
 (segment (start 131.0005 72.4535) (end 131.0005 86.5505) (width 0.5) (layer F.Cu) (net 28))
 (segment (start 131.0005 86.5505) (end 133.1595 88.7095) (width 0.5) (layer F.Cu) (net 28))
 (segment (start 133.1595 88.7095) (end 133.1595 91.313) (width 0.5) (layer F.Cu) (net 28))
 (segment (start 133.1595 91.313) (end 131.7625 92.71) (width 0.5) (layer F.Cu) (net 28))
 (segment (start 131.7625 92.71) (end 125.9205 92.71) (width 0.5) (layer F.Cu) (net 28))
 (segment (start 125.9205 92.71) (end 121.0945 87.884) (width 0.5) (layer F.Cu) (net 28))
 (via (at 117.475 82.3595) (size 0.6) (drill 0.4) (layers F.Cu B.Cu) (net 28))
 (segment (start 121.0945 85.979) (end 117.475 82.3595) (width 0.5) (layer F.Cu) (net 28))
 (segment (start 121.0945 87.884) (end 121.0945 85.979) (width 0.5) (layer F.Cu) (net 28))
 (segment (start 117.445 82.3895) (end 113.9845 82.3895) (width 0.5) (layer B.Cu) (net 28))
 (segment (start 117.475 82.3595) (end 117.445 82.3895) (width 0.5) (layer B.Cu) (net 28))
 (segment (start 168.439999 106.971999) (end 168.439999 107.175199) (width 0.58) (layer B.Cu) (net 18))
 (segment (start 167.64 106.172) (end 168.439999 106.971999) (width 0.58) (layer B.Cu) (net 18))
 (segment (start 168.439999 107.175199) (end 169.1386 107.8738) (width 0.58) (layer B.Cu) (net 18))
 (segment (start 169.1386 107.8738) (end 173.8122 107.8738) (width 0.58) (layer B.Cu) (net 18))
 (segment (start 173.8122 107.8738) (end 174.752 106.934) (width 0.58) (layer B.Cu) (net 18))
 (segment (start 174.752 101.6) (end 172.72 99.568) (width 0.58) (layer B.Cu) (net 18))
 (segment (start 153.7335 49.5895) (end 135.378 67.945) (width 0.25) (layer B.Cu) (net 18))
 (segment (start 153.7335 48.5775) (end 153.7335 49.5895) (width 0.25) (layer B.Cu) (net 18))
 (segment (start 125.349 67.945) (end 120.8405 72.4535) (width 0.25) (layer B.Cu) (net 18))
 (segment (start 135.378 67.945) (end 125.349 67.945) (width 0.25) (layer B.Cu) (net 18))
 (segment (start 120.8405 73.58487) (end 138.75913 91.5035) (width 0.5) (layer B.Cu) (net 18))
 (segment (start 120.8405 72.4535) (end 120.8405 73.58487) (width 0.5) (layer B.Cu) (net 18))
 (segment (start 138.75913 91.5035) (end 181.2925 91.5035) (width 0.5) (layer B.Cu) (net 18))
 (segment (start 181.2925 91.5035) (end 184.404 94.615) (width 0.5) (layer B.Cu) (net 18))
 (segment (start 184.404 94.615) (end 184.404 98.7425) (width 0.5) (layer B.Cu) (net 18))
 (segment (start 181.229 101.9175) (end 174.752 101.9175) (width 0.5) (layer B.Cu) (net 18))
 (segment (start 184.404 98.7425) (end 181.229 101.9175) (width 0.5) (layer B.Cu) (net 18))
 (segment (start 174.752 101.9175) (end 174.752 101.6) (width 0.58) (layer B.Cu) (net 18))
 (segment (start 174.752 106.934) (end 174.752 101.9175) (width 0.58) (layer B.Cu) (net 18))
 (segment (start 125.9205 87.1855) (end 128.4605 89.7255) (width 0.5) (layer F.Cu) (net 31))
 (segment (start 125.9205 72.4535) (end 125.9205 87.1855) (width 0.5) (layer F.Cu) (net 31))
 (segment (start 123.3805 86.6775) (end 126.4285 89.7255) (width 0.5) (layer F.Cu) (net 32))
 (segment (start 123.3805 72.4535) (end 123.3805 86.6775) (width 0.5) (layer F.Cu) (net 32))
 (segment (start 123.1265 65.0875) (end 132.461 65.0875) (width 0.25) (layer B.Cu) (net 34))
 (segment (start 115.7605 72.4535) (end 123.1265 65.0875) (width 0.25) (layer B.Cu) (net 34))
 (segment (start 146.1135 51.435) (end 146.1135 48.5775) (width 0.25) (layer B.Cu) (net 34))
 (segment (start 132.461 65.0875) (end 146.1135 51.435) (width 0.25) (layer B.Cu) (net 34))
 (segment (start 177.000001 100.367999) (end 177.000001 101.231599) (width 0.58) (layer F.Cu) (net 19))
 (segment (start 177.8 99.568) (end 177.000001 100.367999) (width 0.58) (layer F.Cu) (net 19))
 (segment (start 177.000001 101.231599) (end 174.7774 103.4542) (width 0.58) (layer F.Cu) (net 19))
 (segment (start 174.7774 104.1146) (end 172.72 106.172) (width 0.58) (layer F.Cu) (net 19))
 (segment (start 174.7774 103.4542) (end 174.7774 104.1146) (width 0.58) (layer F.Cu) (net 19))
 (segment (start 170.18 106.172) (end 172.72 106.172) (width 0.58) (layer F.Cu) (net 19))
 (segment (start 175.26 99.568) (end 177.8 99.568) (width 0.58) (layer F.Cu) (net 19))
 (segment (start 179.647108 98.768001) (end 181.9275 96.487609) (width 0.5) (layer F.Cu) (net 19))
 (segment (start 178.599999 98.768001) (end 179.647108 98.768001) (width 0.5) (layer F.Cu) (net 19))
 (segment (start 177.8 99.568) (end 178.599999 98.768001) (width 0.5) (layer F.Cu) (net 19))
 (segment (start 181.9275 96.487609) (end 181.9275 73.8505) (width 0.5) (layer F.Cu) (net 19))
 (segment (start 181.9275 73.8505) (end 163.195 55.118) (width 0.5) (layer F.Cu) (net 19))
 (segment (start 148.336 55.118) (end 141.732 48.514) (width 0.5) (layer F.Cu) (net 19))
 (segment (start 163.195 55.118) (end 148.336 55.118) (width 0.5) (layer F.Cu) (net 19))
 (segment (start 123.444 67.31) (end 126.8095 67.31) (width 0.5) (layer F.Cu) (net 33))
 (segment (start 118.3005 72.4535) (end 123.444 67.31) (width 0.5) (layer F.Cu) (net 33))
 (segment (start 139.192 54.9275) (end 139.192 48.514) (width 0.5) (layer F.Cu) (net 33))
 (segment (start 126.8095 67.31) (end 139.192 54.9275) (width 0.5) (layer F.Cu) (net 33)))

